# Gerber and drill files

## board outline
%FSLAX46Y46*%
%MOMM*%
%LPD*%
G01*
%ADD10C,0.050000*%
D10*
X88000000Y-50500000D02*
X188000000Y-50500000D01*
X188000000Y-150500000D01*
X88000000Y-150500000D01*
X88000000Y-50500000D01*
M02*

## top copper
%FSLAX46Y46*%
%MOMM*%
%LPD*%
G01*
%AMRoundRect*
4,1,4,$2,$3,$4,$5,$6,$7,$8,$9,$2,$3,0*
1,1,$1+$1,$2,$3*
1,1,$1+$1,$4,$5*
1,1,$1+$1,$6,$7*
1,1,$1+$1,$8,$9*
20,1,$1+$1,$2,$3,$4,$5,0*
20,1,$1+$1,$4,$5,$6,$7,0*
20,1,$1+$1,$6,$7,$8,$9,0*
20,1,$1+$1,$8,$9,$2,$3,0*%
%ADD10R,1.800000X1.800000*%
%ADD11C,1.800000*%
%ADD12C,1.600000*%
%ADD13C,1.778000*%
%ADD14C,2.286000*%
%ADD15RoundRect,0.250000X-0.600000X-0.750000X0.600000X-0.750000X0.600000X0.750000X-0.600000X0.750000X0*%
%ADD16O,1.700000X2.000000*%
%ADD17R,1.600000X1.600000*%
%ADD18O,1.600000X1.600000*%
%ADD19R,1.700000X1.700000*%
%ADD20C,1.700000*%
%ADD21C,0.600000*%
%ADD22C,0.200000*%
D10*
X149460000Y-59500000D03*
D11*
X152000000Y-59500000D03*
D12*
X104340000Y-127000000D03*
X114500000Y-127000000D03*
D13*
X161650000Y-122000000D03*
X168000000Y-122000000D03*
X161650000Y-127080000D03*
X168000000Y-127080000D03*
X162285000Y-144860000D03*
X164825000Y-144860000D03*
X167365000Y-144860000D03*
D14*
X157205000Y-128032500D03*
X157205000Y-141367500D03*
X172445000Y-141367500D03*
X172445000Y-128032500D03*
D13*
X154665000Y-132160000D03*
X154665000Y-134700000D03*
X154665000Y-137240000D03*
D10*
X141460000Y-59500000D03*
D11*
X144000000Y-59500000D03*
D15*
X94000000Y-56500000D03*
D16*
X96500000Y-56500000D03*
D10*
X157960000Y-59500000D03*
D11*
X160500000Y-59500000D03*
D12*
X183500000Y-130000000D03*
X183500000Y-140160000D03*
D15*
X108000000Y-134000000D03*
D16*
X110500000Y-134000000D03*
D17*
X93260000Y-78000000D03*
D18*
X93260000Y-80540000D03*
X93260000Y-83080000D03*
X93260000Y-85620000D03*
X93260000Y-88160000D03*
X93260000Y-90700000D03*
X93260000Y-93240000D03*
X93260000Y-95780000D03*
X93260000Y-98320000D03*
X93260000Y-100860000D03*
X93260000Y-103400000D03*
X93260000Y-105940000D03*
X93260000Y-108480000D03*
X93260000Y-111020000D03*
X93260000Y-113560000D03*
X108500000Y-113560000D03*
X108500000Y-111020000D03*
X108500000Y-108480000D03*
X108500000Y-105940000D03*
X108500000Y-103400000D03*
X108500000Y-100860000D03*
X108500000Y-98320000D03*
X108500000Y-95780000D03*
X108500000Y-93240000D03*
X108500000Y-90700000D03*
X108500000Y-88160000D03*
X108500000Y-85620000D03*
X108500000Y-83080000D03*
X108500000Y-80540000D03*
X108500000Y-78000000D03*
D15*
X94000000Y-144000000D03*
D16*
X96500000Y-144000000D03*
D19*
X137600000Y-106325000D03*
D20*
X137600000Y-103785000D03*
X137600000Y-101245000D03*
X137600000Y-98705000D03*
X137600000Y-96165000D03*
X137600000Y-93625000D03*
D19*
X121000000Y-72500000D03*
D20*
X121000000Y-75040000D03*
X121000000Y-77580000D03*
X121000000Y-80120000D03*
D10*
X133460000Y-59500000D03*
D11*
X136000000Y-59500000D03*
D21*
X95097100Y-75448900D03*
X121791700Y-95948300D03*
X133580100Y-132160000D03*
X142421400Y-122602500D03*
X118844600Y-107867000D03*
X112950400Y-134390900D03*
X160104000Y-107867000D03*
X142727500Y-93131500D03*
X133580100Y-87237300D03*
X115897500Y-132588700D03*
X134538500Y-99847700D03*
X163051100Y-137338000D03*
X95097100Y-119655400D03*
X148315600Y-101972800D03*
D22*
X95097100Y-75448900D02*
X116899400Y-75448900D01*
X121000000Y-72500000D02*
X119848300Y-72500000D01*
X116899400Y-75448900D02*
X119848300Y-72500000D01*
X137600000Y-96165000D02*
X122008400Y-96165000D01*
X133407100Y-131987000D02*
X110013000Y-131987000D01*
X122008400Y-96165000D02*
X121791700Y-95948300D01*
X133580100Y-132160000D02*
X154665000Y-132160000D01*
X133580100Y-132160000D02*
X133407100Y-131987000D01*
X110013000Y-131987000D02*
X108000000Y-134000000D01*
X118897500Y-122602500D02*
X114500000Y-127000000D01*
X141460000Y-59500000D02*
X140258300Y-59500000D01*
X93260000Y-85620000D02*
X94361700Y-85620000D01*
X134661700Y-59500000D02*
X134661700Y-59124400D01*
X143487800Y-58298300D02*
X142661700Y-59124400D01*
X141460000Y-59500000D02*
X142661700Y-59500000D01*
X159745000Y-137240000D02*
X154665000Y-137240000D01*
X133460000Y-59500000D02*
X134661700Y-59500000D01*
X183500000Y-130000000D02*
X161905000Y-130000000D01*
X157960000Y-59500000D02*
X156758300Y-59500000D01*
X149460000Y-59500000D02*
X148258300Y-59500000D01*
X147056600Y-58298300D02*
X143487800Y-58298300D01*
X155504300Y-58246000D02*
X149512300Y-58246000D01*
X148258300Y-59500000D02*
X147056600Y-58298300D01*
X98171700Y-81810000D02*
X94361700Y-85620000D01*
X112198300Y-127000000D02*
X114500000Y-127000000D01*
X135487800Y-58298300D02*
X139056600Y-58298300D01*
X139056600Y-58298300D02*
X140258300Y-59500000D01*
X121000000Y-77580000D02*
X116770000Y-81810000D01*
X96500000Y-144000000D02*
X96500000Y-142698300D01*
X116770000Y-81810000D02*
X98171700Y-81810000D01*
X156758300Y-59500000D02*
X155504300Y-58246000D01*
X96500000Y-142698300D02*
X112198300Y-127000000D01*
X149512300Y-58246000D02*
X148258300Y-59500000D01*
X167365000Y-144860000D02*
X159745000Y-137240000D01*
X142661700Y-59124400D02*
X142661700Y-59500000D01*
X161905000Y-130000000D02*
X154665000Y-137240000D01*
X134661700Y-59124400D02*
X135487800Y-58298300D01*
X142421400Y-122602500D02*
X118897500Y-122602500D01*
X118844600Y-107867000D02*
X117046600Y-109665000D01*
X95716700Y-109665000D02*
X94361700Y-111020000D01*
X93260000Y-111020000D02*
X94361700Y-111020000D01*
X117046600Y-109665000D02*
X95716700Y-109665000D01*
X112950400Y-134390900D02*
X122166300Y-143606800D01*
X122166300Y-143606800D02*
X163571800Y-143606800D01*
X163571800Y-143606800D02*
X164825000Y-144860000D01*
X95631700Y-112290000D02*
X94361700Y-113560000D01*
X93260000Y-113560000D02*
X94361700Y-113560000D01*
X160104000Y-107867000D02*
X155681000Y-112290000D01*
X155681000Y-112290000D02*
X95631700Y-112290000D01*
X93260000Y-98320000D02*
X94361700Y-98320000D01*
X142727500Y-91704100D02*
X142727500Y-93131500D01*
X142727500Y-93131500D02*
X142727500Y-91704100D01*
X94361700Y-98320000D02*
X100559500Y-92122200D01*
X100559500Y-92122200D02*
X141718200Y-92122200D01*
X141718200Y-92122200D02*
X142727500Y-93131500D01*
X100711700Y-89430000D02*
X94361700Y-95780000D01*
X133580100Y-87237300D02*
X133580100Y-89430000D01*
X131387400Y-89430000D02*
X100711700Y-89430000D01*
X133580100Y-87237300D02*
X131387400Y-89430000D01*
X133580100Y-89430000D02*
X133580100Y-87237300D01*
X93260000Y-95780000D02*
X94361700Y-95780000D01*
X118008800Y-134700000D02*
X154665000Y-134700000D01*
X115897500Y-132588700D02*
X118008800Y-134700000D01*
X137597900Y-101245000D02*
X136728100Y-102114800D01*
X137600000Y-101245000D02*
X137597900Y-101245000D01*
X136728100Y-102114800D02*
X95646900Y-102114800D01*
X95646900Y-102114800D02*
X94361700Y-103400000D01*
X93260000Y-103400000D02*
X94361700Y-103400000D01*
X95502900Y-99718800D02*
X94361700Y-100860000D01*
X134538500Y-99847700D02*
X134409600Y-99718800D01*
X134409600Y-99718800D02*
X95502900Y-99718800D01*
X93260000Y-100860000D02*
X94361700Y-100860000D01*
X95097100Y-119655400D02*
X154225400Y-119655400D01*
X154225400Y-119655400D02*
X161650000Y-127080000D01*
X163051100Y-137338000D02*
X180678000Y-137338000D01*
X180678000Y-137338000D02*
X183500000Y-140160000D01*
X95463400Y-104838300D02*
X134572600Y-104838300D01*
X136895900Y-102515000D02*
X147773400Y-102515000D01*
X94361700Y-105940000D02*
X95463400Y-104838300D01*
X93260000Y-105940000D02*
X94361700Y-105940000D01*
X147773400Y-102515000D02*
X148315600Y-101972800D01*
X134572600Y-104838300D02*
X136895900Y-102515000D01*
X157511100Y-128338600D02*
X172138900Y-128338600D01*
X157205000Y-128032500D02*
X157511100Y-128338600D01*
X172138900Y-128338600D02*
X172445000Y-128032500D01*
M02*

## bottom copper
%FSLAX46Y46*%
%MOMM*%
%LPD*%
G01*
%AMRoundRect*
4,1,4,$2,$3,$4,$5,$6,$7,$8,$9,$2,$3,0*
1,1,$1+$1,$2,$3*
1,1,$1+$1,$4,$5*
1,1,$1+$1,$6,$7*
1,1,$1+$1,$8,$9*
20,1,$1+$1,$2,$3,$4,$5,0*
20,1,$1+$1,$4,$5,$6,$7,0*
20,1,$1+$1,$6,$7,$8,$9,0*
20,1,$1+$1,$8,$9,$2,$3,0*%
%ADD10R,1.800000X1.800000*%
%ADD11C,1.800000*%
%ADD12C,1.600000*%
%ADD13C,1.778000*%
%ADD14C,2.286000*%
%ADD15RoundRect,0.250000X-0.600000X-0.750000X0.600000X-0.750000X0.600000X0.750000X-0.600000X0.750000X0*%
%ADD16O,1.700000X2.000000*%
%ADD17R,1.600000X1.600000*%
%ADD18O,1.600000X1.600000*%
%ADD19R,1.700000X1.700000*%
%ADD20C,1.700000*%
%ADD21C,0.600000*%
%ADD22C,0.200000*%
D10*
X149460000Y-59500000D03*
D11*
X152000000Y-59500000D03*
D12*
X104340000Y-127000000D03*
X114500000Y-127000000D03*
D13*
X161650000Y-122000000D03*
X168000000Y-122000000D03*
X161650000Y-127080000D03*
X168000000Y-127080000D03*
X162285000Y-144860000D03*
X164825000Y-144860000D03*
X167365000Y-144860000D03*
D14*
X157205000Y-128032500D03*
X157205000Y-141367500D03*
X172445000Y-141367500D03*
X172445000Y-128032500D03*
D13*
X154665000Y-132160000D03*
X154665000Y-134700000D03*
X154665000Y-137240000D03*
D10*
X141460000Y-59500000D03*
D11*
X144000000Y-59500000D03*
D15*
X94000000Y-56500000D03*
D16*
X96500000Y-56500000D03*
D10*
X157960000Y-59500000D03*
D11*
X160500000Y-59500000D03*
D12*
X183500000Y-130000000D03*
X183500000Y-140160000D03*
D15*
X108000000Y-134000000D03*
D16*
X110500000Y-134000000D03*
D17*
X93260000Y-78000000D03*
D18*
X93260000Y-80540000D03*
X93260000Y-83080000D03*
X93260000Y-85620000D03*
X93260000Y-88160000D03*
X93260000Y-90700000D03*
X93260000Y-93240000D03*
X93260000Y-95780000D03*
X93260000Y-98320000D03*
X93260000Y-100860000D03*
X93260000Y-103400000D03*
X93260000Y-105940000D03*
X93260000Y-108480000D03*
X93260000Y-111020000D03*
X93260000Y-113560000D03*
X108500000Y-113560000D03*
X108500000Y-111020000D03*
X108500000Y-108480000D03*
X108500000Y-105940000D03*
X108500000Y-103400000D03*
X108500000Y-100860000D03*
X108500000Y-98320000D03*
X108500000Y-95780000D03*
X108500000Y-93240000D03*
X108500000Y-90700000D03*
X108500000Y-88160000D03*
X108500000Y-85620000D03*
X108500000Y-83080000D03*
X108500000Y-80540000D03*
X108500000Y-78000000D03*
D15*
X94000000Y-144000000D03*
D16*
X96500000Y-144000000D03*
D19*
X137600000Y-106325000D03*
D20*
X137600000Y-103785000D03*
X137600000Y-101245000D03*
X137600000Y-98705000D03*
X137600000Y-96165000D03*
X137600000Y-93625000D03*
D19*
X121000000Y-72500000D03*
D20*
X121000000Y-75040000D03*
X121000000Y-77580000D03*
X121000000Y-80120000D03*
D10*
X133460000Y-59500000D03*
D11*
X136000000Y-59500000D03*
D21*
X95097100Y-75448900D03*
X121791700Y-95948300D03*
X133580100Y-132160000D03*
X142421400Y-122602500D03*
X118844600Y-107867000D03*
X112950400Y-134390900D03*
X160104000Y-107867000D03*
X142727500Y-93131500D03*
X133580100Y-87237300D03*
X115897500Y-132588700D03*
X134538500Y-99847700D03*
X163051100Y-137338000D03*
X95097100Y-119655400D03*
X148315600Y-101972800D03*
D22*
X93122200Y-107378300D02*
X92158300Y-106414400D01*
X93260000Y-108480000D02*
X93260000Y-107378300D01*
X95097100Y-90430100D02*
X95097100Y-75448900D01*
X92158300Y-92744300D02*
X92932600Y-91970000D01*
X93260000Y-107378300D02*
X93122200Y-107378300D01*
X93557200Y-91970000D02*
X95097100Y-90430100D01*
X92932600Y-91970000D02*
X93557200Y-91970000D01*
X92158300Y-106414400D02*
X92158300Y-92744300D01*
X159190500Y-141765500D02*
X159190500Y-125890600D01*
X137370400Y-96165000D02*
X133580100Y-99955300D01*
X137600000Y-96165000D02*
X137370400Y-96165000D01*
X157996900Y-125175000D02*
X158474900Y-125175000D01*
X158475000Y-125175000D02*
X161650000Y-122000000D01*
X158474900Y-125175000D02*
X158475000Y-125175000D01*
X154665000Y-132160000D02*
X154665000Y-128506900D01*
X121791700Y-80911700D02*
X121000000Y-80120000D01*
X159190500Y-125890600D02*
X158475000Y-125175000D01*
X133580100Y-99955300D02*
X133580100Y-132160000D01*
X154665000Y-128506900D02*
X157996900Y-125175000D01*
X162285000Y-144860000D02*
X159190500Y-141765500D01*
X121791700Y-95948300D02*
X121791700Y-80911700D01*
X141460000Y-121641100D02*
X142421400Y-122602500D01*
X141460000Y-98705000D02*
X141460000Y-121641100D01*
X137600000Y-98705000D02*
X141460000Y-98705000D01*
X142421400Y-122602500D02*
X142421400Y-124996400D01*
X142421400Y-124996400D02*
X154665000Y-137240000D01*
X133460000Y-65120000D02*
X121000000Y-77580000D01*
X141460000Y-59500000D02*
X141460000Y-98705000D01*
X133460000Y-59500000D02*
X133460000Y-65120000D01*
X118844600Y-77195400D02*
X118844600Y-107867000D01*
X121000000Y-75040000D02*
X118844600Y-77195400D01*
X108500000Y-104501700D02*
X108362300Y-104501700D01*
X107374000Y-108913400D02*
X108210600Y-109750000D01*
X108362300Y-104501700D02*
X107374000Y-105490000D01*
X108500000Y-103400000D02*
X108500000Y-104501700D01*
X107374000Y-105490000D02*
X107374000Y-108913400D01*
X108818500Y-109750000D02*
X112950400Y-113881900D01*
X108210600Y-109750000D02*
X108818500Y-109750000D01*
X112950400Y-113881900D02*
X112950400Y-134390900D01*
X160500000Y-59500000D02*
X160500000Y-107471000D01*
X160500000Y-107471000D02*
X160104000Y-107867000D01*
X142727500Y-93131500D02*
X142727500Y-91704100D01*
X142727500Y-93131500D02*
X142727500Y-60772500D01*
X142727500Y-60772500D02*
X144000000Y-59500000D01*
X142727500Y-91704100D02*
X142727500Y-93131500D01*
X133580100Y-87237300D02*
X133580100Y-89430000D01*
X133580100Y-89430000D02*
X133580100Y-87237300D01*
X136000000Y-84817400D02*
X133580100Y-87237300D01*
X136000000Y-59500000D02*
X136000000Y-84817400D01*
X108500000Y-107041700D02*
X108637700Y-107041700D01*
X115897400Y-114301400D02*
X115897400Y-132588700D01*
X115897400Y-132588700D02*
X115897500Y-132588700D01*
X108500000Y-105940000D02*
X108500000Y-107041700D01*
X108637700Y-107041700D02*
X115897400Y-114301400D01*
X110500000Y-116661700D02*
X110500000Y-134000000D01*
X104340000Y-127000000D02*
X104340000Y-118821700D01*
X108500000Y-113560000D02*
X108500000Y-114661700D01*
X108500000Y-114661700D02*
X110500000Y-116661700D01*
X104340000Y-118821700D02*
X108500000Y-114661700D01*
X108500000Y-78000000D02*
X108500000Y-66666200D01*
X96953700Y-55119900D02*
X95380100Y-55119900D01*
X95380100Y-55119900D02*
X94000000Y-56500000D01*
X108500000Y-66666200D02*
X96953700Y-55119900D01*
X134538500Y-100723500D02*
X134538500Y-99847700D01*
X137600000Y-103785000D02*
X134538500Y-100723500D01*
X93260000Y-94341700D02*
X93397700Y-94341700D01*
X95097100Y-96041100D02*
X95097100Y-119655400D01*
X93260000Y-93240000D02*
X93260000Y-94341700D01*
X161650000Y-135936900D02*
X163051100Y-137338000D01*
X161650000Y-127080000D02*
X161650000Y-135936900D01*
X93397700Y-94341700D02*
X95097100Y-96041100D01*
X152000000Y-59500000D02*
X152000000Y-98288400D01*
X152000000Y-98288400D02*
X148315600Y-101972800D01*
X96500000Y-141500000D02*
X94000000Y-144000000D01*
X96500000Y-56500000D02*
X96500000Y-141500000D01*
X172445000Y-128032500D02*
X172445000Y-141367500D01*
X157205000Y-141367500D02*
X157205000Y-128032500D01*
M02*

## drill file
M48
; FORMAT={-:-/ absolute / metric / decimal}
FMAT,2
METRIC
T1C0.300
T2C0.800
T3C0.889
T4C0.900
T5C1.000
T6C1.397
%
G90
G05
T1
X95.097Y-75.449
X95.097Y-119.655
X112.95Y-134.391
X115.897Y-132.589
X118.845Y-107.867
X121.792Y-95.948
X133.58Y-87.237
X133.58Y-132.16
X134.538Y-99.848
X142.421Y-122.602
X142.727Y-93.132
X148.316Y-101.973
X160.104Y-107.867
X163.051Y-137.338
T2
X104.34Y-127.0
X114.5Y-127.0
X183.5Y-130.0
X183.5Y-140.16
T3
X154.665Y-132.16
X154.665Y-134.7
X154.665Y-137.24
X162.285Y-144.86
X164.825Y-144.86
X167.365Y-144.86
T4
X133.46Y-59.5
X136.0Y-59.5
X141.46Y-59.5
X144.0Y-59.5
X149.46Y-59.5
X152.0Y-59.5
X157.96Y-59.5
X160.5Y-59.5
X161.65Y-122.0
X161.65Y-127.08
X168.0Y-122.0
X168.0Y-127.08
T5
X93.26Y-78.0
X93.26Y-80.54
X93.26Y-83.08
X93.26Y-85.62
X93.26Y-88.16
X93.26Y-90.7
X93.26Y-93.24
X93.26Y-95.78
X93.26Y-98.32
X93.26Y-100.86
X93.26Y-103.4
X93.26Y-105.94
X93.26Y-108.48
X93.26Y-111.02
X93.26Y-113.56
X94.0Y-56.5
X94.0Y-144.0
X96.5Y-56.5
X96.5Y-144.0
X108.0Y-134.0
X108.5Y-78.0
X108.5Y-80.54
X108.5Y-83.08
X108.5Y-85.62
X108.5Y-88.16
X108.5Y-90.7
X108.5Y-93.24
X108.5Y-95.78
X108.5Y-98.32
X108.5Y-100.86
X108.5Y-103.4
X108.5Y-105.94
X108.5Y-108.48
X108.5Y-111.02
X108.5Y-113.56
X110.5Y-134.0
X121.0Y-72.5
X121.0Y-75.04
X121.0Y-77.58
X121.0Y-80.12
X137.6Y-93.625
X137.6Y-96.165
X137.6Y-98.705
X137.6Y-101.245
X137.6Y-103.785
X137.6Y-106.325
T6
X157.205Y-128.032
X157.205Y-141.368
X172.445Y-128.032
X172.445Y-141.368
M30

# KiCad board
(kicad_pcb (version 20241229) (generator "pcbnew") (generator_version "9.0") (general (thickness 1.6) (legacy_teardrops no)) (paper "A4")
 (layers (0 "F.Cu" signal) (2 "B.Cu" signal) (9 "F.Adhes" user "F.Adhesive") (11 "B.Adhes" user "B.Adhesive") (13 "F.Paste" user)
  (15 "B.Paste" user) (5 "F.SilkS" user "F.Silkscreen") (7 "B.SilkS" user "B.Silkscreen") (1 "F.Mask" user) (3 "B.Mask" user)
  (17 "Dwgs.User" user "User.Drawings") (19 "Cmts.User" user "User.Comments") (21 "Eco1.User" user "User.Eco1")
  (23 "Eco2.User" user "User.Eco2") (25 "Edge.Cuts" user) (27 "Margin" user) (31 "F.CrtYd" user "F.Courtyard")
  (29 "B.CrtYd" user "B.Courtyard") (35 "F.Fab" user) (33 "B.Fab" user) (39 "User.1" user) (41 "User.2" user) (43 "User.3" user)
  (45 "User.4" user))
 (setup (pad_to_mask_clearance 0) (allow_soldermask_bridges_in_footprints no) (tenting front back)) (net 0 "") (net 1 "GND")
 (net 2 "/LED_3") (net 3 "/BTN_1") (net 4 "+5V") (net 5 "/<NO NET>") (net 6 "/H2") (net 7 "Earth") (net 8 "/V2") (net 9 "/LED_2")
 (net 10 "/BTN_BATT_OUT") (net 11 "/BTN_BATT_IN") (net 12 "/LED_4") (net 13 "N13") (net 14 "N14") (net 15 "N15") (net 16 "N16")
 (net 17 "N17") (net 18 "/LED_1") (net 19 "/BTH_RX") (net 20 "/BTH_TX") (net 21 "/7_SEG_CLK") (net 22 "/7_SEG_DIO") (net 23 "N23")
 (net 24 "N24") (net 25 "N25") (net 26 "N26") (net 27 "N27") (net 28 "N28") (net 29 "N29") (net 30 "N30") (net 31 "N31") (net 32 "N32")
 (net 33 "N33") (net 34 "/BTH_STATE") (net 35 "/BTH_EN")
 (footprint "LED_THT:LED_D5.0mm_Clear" (layer "F.Cu") (at 149.46 59.5)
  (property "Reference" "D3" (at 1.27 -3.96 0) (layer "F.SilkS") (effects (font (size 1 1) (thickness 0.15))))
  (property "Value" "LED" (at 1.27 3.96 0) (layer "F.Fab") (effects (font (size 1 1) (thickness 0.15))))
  (pad "1" thru_hole rect (at 0 0) (size 1.8 1.8) (drill 0.9) (layers "*.Cu" "*.Mask") (remove_unused_layers no) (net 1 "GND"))
  (pad "2" thru_hole circle (at 2.54 0) (size 1.8 1.8) (drill 0.9) (layers "*.Cu" "*.Mask") (remove_unused_layers no) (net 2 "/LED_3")))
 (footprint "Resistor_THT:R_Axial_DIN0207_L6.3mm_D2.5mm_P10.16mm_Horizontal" (layer "F.Cu") (at 104.34 127)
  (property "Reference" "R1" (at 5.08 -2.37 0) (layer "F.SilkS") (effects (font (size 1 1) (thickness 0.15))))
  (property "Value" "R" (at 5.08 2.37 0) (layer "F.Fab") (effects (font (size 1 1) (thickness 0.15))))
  (pad "1" thru_hole circle (at 0 0) (size 1.6 1.6) (drill 0.8) (layers "*.Cu" "*.Mask") (remove_unused_layers no) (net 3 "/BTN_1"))
  (pad "2" thru_hole circle (at 10.16 0) (size 1.6 1.6) (drill 0.8) (layers "*.Cu" "*.Mask") (remove_unused_layers no) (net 1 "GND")))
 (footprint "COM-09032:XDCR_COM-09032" (layer "F.Cu") (at 164.825 134.7)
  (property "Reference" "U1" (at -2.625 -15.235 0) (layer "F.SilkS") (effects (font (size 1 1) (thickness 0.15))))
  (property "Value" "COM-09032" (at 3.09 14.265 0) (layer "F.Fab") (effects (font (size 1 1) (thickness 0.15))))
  (pad "B1A" thru_hole circle (at -3.175 -12.7) (size 1.778 1.778) (drill 0.9) (layers "*.Cu" "*.Mask") (remove_unused_layers no)
   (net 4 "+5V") (solder_mask_margin 0.102))
  (pad "B1B" thru_hole circle (at 3.175 -12.7) (size 1.778 1.778) (drill 0.9) (layers "*.Cu" "*.Mask") (remove_unused_layers no)
   (solder_mask_margin 0.102))
  (pad "B2A" thru_hole circle (at -3.175 -7.62) (size 1.778 1.778) (drill 0.9) (layers "*.Cu" "*.Mask") (remove_unused_layers no)
   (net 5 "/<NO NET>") (solder_mask_margin 0.102))
  (pad "B2B" thru_hole circle (at 3.175 -7.62) (size 1.778 1.778) (drill 0.9) (layers "*.Cu" "*.Mask") (remove_unused_layers no)
   (solder_mask_margin 0.102))
  (pad "H1" thru_hole circle (at -2.54 10.16) (size 1.778 1.778) (drill 0.889) (layers "*.Cu" "*.Mask") (remove_unused_layers no)
   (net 4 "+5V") (solder_mask_margin 0.102))
  (pad "H2" thru_hole circle (at 0 10.16) (size 1.778 1.778) (drill 0.889) (layers "*.Cu" "*.Mask") (remove_unused_layers no) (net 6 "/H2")
   (solder_mask_margin 0.102))
  (pad "H3" thru_hole circle (at 2.54 10.16) (size 1.778 1.778) (drill 0.889) (layers "*.Cu" "*.Mask") (remove_unused_layers no)
   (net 1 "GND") (solder_mask_margin 0.102))
  (pad "S1" thru_hole circle (at -7.62 -6.6675) (size 2.286 2.286) (drill 1.397) (layers "*.Cu" "*.Mask") (remove_unused_layers no)
   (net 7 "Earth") (solder_mask_margin 0.102))
  (pad "S2" thru_hole circle (at -7.62 6.6675) (size 2.286 2.286) (drill 1.397) (layers "*.Cu" "*.Mask") (remove_unused_layers no)
   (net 7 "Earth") (solder_mask_margin 0.102))
  (pad "S3" thru_hole circle (at 7.62 6.6675) (size 2.286 2.286) (drill 1.397) (layers "*.Cu" "*.Mask") (remove_unused_layers no)
   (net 7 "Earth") (solder_mask_margin 0.102))
  (pad "S4" thru_hole circle (at 7.62 -6.6675) (size 2.286 2.286) (drill 1.397) (layers "*.Cu" "*.Mask") (remove_unused_layers no)
   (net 7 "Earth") (solder_mask_margin 0.102))
  (pad "V1" thru_hole circle (at -10.16 -2.54) (size 1.778 1.778) (drill 0.889) (layers "*.Cu" "*.Mask") (remove_unused_layers no)
   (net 4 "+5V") (solder_mask_margin 0.102))
  (pad "V2" thru_hole circle (at -10.16 0) (size 1.778 1.778) (drill 0.889) (layers "*.Cu" "*.Mask") (remove_unused_layers no) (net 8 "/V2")
   (solder_mask_margin 0.102))
  (pad "V3" thru_hole circle (at -10.16 2.54) (size 1.778 1.778) (drill 0.889) (layers "*.Cu" "*.Mask") (remove_unused_layers no)
   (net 1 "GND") (solder_mask_margin 0.102)))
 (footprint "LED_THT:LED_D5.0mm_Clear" (layer "F.Cu") (at 141.46 59.5)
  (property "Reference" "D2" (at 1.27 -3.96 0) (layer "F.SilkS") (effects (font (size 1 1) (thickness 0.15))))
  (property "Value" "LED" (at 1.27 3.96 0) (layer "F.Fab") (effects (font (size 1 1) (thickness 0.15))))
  (pad "1" thru_hole rect (at 0 0) (size 1.8 1.8) (drill 0.9) (layers "*.Cu" "*.Mask") (remove_unused_layers no) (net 1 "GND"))
  (pad "2" thru_hole circle (at 2.54 0) (size 1.8 1.8) (drill 0.9) (layers "*.Cu" "*.Mask") (remove_unused_layers no) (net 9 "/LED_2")))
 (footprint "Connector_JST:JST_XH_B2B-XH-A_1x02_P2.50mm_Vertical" (layer "F.Cu") (at 94 56.5)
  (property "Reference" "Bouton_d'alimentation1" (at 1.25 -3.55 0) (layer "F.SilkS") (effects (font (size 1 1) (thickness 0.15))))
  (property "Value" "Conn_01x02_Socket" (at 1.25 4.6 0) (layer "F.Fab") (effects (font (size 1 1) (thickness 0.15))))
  (pad "1" thru_hole roundrect (at 0 0) (size 1.7 2) (drill 1) (layers "*.Cu" "*.Mask") (remove_unused_layers no)
   (roundrect_rratio 0.147059) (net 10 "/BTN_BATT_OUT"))
  (pad "2" thru_hole oval (at 2.5 0) (size 1.7 2) (drill 1) (layers "*.Cu" "*.Mask") (remove_unused_layers no) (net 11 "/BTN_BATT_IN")))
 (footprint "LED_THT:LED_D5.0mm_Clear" (layer "F.Cu") (at 157.96 59.5)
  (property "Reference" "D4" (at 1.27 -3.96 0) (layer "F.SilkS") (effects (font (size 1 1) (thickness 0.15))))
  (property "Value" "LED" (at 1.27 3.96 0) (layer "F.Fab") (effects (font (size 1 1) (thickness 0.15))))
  (pad "1" thru_hole rect (at 0 0) (size 1.8 1.8) (drill 0.9) (layers "*.Cu" "*.Mask") (remove_unused_layers no) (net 1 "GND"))
  (pad "2" thru_hole circle (at 2.54 0) (size 1.8 1.8) (drill 0.9) (layers "*.Cu" "*.Mask") (remove_unused_layers no) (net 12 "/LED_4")))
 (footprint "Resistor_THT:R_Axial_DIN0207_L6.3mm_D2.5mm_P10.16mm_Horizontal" (layer "F.Cu") (at 183.5 130 -90)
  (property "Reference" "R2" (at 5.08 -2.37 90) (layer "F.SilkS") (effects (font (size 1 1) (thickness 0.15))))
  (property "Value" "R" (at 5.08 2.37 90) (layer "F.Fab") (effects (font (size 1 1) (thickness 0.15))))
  (pad "1" thru_hole circle (at 0 0 270) (size 1.6 1.6) (drill 0.8) (layers "*.Cu" "*.Mask") (remove_unused_layers no) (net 1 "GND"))
  (pad "2" thru_hole circle (at 10.16 0 270) (size 1.6 1.6) (drill 0.8) (layers "*.Cu" "*.Mask") (remove_unused_layers no)
   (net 5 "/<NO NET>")))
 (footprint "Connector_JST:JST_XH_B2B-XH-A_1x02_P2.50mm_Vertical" (layer "F.Cu") (at 108 134)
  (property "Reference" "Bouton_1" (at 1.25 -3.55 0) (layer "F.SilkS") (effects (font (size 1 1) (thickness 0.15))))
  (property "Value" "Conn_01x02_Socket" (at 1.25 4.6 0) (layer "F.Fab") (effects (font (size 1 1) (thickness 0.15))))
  (pad "1" thru_hole roundrect (at 0 0) (size 1.7 2) (drill 1) (layers "*.Cu" "*.Mask") (remove_unused_layers no)
   (roundrect_rratio 0.147059) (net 4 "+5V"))
  (pad "2" thru_hole oval (at 2.5 0) (size 1.7 2) (drill 1) (layers "*.Cu" "*.Mask") (remove_unused_layers no) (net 3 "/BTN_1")))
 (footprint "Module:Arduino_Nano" (layer "F.Cu") (at 93.26 78)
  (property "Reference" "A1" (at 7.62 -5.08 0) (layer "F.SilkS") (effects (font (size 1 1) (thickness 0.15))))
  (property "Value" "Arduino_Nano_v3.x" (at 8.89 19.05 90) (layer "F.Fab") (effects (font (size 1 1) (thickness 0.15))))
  (pad "1" thru_hole rect (at 0 0) (size 1.6 1.6) (drill 1) (layers "*.Cu" "*.Mask") (remove_unused_layers no) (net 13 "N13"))
  (pad "2" thru_hole oval (at 0 2.54) (size 1.6 1.6) (drill 1) (layers "*.Cu" "*.Mask") (remove_unused_layers no) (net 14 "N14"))
  (pad "3" thru_hole oval (at 0 5.08) (size 1.6 1.6) (drill 1) (layers "*.Cu" "*.Mask") (remove_unused_layers no) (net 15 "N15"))
  (pad "4" thru_hole oval (at 0 7.62) (size 1.6 1.6) (drill 1) (layers "*.Cu" "*.Mask") (remove_unused_layers no) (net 1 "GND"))
  (pad "5" thru_hole oval (at 0 10.16) (size 1.6 1.6) (drill 1) (layers "*.Cu" "*.Mask") (remove_unused_layers no) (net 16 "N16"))
  (pad "6" thru_hole oval (at 0 12.7) (size 1.6 1.6) (drill 1) (layers "*.Cu" "*.Mask") (remove_unused_layers no) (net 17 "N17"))
  (pad "7" thru_hole oval (at 0 15.24) (size 1.6 1.6) (drill 1) (layers "*.Cu" "*.Mask") (remove_unused_layers no) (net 5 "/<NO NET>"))
  (pad "8" thru_hole oval (at 0 17.78) (size 1.6 1.6) (drill 1) (layers "*.Cu" "*.Mask") (remove_unused_layers no) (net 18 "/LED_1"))
  (pad "9" thru_hole oval (at 0 20.32) (size 1.6 1.6) (drill 1) (layers "*.Cu" "*.Mask") (remove_unused_layers no) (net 9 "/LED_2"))
  (pad "10" thru_hole oval (at 0 22.86) (size 1.6 1.6) (drill 1) (layers "*.Cu" "*.Mask") (remove_unused_layers no) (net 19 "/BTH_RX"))
  (pad "11" thru_hole oval (at 0 25.4) (size 1.6 1.6) (drill 1) (layers "*.Cu" "*.Mask") (remove_unused_layers no) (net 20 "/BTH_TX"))
  (pad "12" thru_hole oval (at 0 27.94) (size 1.6 1.6) (drill 1) (layers "*.Cu" "*.Mask") (remove_unused_layers no) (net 2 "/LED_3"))
  (pad "13" thru_hole oval (at 0 30.48) (size 1.6 1.6) (drill 1) (layers "*.Cu" "*.Mask") (remove_unused_layers no) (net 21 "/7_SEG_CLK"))
  (pad "14" thru_hole oval (at 0 33.02) (size 1.6 1.6) (drill 1) (layers "*.Cu" "*.Mask") (remove_unused_layers no) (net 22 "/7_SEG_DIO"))
  (pad "15" thru_hole oval (at 0 35.56) (size 1.6 1.6) (drill 1) (layers "*.Cu" "*.Mask") (remove_unused_layers no) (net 12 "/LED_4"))
  (pad "16" thru_hole oval (at 15.24 35.56) (size 1.6 1.6) (drill 1) (layers "*.Cu" "*.Mask") (remove_unused_layers no) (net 3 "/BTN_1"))
  (pad "17" thru_hole oval (at 15.24 33.02) (size 1.6 1.6) (drill 1) (layers "*.Cu" "*.Mask") (remove_unused_layers no) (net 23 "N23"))
  (pad "18" thru_hole oval (at 15.24 30.48) (size 1.6 1.6) (drill 1) (layers "*.Cu" "*.Mask") (remove_unused_layers no) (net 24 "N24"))
  (pad "19" thru_hole oval (at 15.24 27.94) (size 1.6 1.6) (drill 1) (layers "*.Cu" "*.Mask") (remove_unused_layers no) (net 8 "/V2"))
  (pad "20" thru_hole oval (at 15.24 25.4) (size 1.6 1.6) (drill 1) (layers "*.Cu" "*.Mask") (remove_unused_layers no) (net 6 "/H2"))
  (pad "21" thru_hole oval (at 15.24 22.86) (size 1.6 1.6) (drill 1) (layers "*.Cu" "*.Mask") (remove_unused_layers no) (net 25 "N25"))
  (pad "22" thru_hole oval (at 15.24 20.32) (size 1.6 1.6) (drill 1) (layers "*.Cu" "*.Mask") (remove_unused_layers no) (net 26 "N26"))
  (pad "23" thru_hole oval (at 15.24 17.78) (size 1.6 1.6) (drill 1) (layers "*.Cu" "*.Mask") (remove_unused_layers no) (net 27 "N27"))
  (pad "24" thru_hole oval (at 15.24 15.24) (size 1.6 1.6) (drill 1) (layers "*.Cu" "*.Mask") (remove_unused_layers no) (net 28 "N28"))
  (pad "25" thru_hole oval (at 15.24 12.7) (size 1.6 1.6) (drill 1) (layers "*.Cu" "*.Mask") (remove_unused_layers no) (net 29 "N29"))
  (pad "26" thru_hole oval (at 15.24 10.16) (size 1.6 1.6) (drill 1) (layers "*.Cu" "*.Mask") (remove_unused_layers no) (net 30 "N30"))
  (pad "27" thru_hole oval (at 15.24 7.62) (size 1.6 1.6) (drill 1) (layers "*.Cu" "*.Mask") (remove_unused_layers no) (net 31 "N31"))
  (pad "28" thru_hole oval (at 15.24 5.08) (size 1.6 1.6) (drill 1) (layers "*.Cu" "*.Mask") (remove_unused_layers no) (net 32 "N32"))
  (pad "29" thru_hole oval (at 15.24 2.54) (size 1.6 1.6) (drill 1) (layers "*.Cu" "*.Mask") (remove_unused_layers no) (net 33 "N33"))
  (pad "30" thru_hole oval (at 15.24 0) (size 1.6 1.6) (drill 1) (layers "*.Cu" "*.Mask") (remove_unused_layers no) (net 10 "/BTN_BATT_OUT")))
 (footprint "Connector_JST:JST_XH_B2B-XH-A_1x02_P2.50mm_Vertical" (layer "F.Cu") (at 94 144)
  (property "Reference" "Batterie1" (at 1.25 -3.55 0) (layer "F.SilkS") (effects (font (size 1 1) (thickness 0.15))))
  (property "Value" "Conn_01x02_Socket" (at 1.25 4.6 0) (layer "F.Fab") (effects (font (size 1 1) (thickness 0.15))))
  (pad "1" thru_hole roundrect (at 0 0) (size 1.7 2) (drill 1) (layers "*.Cu" "*.Mask") (remove_unused_layers no)
   (roundrect_rratio 0.147059) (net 11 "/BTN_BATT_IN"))
  (pad "2" thru_hole oval (at 2.5 0) (size 1.7 2) (drill 1) (layers "*.Cu" "*.Mask") (remove_unused_layers no) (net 1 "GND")))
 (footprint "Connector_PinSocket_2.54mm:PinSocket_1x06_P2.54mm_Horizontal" (layer "F.Cu") (at 137.6 106.325 180)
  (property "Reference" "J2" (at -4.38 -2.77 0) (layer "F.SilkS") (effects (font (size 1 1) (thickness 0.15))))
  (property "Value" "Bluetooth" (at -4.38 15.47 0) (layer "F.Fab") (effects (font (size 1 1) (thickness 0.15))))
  (pad "1" thru_hole rect (at 0 0 180) (size 1.7 1.7) (drill 1) (layers "*.Cu" "*.Mask") (remove_unused_layers no) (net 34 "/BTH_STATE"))
  (pad "2" thru_hole circle (at 0 2.54 180) (size 1.7 1.7) (drill 1) (layers "*.Cu" "*.Mask") (remove_unused_layers no) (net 19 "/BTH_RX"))
  (pad "3" thru_hole circle (at 0 5.08 180) (size 1.7 1.7) (drill 1) (layers "*.Cu" "*.Mask") (remove_unused_layers no) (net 20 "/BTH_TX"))
  (pad "4" thru_hole circle (at 0 7.62 180) (size 1.7 1.7) (drill 1) (layers "*.Cu" "*.Mask") (remove_unused_layers no) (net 1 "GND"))
  (pad "5" thru_hole circle (at 0 10.16 180) (size 1.7 1.7) (drill 1) (layers "*.Cu" "*.Mask") (remove_unused_layers no) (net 4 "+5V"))
  (pad "6" thru_hole circle (at 0 12.7 180) (size 1.7 1.7) (drill 1) (layers "*.Cu" "*.Mask") (remove_unused_layers no) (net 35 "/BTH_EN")))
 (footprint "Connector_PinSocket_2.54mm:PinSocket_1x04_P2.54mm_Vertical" (layer "F.Cu") (at 121 72.5)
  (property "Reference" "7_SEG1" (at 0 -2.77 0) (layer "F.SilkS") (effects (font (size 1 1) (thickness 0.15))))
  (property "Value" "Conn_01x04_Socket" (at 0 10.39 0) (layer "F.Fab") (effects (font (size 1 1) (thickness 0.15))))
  (pad "1" thru_hole rect (at 0 0) (size 1.7 1.7) (drill 1) (layers "*.Cu" "*.Mask") (remove_unused_layers no) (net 21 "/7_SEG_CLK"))
  (pad "2" thru_hole circle (at 0 2.54) (size 1.7 1.7) (drill 1) (layers "*.Cu" "*.Mask") (remove_unused_layers no) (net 22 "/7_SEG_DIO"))
  (pad "3" thru_hole circle (at 0 5.08) (size 1.7 1.7) (drill 1) (layers "*.Cu" "*.Mask") (remove_unused_layers no) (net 1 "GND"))
  (pad "4" thru_hole circle (at 0 7.62) (size 1.7 1.7) (drill 1) (layers "*.Cu" "*.Mask") (remove_unused_layers no) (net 4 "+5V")))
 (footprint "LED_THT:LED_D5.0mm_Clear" (layer "F.Cu") (at 133.46 59.5)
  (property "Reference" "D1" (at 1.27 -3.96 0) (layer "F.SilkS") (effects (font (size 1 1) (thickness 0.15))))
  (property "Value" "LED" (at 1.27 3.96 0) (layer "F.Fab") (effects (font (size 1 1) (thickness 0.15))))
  (pad "1" thru_hole rect (at 0 0) (size 1.8 1.8) (drill 0.9) (layers "*.Cu" "*.Mask") (remove_unused_layers no) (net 1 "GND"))
  (pad "2" thru_hole circle (at 2.54 0) (size 1.8 1.8) (drill 0.9) (layers "*.Cu" "*.Mask") (remove_unused_layers no) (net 18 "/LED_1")))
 (gr_rect (start 88 50.5) (end 188 150.5) (stroke (width 0.05) (type solid)) (fill no) (layer "Edge.Cuts"))
 (segment (start 95.0971 75.4489) (end 116.8994 75.4489) (width 0.2) (layer "F.Cu") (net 21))
 (segment (start 121 72.5) (end 119.8483 72.5) (width 0.2) (layer "F.Cu") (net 21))
 (segment (start 116.8994 75.4489) (end 119.8483 72.5) (width 0.2) (layer "F.Cu") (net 21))
 (via (at 95.0971 75.4489) (size 0.6) (drill 0.3) (layers "F.Cu" "B.Cu") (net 21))
 (segment (start 93.1222 107.3783) (end 92.1583 106.4144) (width 0.2) (layer "B.Cu") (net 21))
 (segment (start 93.26 108.48) (end 93.26 107.3783) (width 0.2) (layer "B.Cu") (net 21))
 (segment (start 95.0971 90.4301) (end 95.0971 75.4489) (width 0.2) (layer "B.Cu") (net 21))
 (segment (start 92.1583 92.7443) (end 92.9326 91.97) (width 0.2) (layer "B.Cu") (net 21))
 (segment (start 93.26 107.3783) (end 93.1222 107.3783) (width 0.2) (layer "B.Cu") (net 21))
 (segment (start 93.5572 91.97) (end 95.0971 90.4301) (width 0.2) (layer "B.Cu") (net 21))
 (segment (start 92.9326 91.97) (end 93.5572 91.97) (width 0.2) (layer "B.Cu") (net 21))
 (segment (start 92.1583 106.4144) (end 92.1583 92.7443) (width 0.2) (layer "B.Cu") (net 21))
 (segment (start 137.6 96.165) (end 122.0084 96.165) (width 0.2) (layer "F.Cu") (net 4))
 (segment (start 133.4071 131.987) (end 110.013 131.987) (width 0.2) (layer "F.Cu") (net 4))
 (segment (start 122.0084 96.165) (end 121.7917 95.9483) (width 0.2) (layer "F.Cu") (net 4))
 (segment (start 133.5801 132.16) (end 154.665 132.16) (width 0.2) (layer "F.Cu") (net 4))
 (segment (start 133.5801 132.16) (end 133.4071 131.987) (width 0.2) (layer "F.Cu") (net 4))
 (segment (start 110.013 131.987) (end 108 134) (width 0.2) (layer "F.Cu") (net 4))
 (via (at 121.7917 95.9483) (size 0.6) (drill 0.3) (layers "F.Cu" "B.Cu") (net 4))
 (via (at 133.5801 132.16) (size 0.6) (drill 0.3) (layers "F.Cu" "B.Cu") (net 4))
 (segment (start 159.1905 141.7655) (end 159.1905 125.8906) (width 0.2) (layer "B.Cu") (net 4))
 (segment (start 137.3704 96.165) (end 133.5801 99.9553) (width 0.2) (layer "B.Cu") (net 4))
 (segment (start 137.6 96.165) (end 137.3704 96.165) (width 0.2) (layer "B.Cu") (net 4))
 (segment (start 157.9969 125.175) (end 158.4749 125.175) (width 0.2) (layer "B.Cu") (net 4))
 (segment (start 158.475 125.175) (end 161.65 122) (width 0.2) (layer "B.Cu") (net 4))
 (segment (start 158.4749 125.175) (end 158.475 125.175) (width 0.2) (layer "B.Cu") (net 4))
 (segment (start 154.665 132.16) (end 154.665 128.5069) (width 0.2) (layer "B.Cu") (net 4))
 (segment (start 121.7917 80.9117) (end 121 80.12) (width 0.2) (layer "B.Cu") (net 4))
 (segment (start 159.1905 125.8906) (end 158.475 125.175) (width 0.2) (layer "B.Cu") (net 4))
 (segment (start 133.5801 99.9553) (end 133.5801 132.16) (width 0.2) (layer "B.Cu") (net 4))
 (segment (start 154.665 128.5069) (end 157.9969 125.175) (width 0.2) (layer "B.Cu") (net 4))
 (segment (start 162.285 144.86) (end 159.1905 141.7655) (width 0.2) (layer "B.Cu") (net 4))
 (segment (start 121.7917 95.9483) (end 121.7917 80.9117) (width 0.2) (layer "B.Cu") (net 4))
 (segment (start 118.8975 122.6025) (end 114.5 127) (width 0.2) (layer "F.Cu") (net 1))
 (segment (start 141.46 59.5) (end 140.2583 59.5) (width 0.2) (layer "F.Cu") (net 1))
 (segment (start 93.26 85.62) (end 94.3617 85.62) (width 0.2) (layer "F.Cu") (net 1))
 (segment (start 134.6617 59.5) (end 134.6617 59.1244) (width 0.2) (layer "F.Cu") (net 1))
 (segment (start 143.4878 58.2983) (end 142.6617 59.1244) (width 0.2) (layer "F.Cu") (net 1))
 (segment (start 141.46 59.5) (end 142.6617 59.5) (width 0.2) (layer "F.Cu") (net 1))
 (segment (start 159.745 137.24) (end 154.665 137.24) (width 0.2) (layer "F.Cu") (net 1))
 (segment (start 133.46 59.5) (end 134.6617 59.5) (width 0.2) (layer "F.Cu") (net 1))
 (segment (start 183.5 130) (end 161.905 130) (width 0.2) (layer "F.Cu") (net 1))
 (segment (start 157.96 59.5) (end 156.7583 59.5) (width 0.2) (layer "F.Cu") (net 1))
 (segment (start 149.46 59.5) (end 148.2583 59.5) (width 0.2) (layer "F.Cu") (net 1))
 (segment (start 147.0566 58.2983) (end 143.4878 58.2983) (width 0.2) (layer "F.Cu") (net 1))
 (segment (start 155.5043 58.246) (end 149.5123 58.246) (width 0.2) (layer "F.Cu") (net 1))
 (segment (start 148.2583 59.5) (end 147.0566 58.2983) (width 0.2) (layer "F.Cu") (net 1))
 (segment (start 98.1717 81.81) (end 94.3617 85.62) (width 0.2) (layer "F.Cu") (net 1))
 (segment (start 112.1983 127) (end 114.5 127) (width 0.2) (layer "F.Cu") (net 1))
 (segment (start 135.4878 58.2983) (end 139.0566 58.2983) (width 0.2) (layer "F.Cu") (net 1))
 (segment (start 139.0566 58.2983) (end 140.2583 59.5) (width 0.2) (layer "F.Cu") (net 1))
 (segment (start 121 77.58) (end 116.77 81.81) (width 0.2) (layer "F.Cu") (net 1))
 (segment (start 96.5 144) (end 96.5 142.6983) (width 0.2) (layer "F.Cu") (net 1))
 (segment (start 116.77 81.81) (end 98.1717 81.81) (width 0.2) (layer "F.Cu") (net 1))
 (segment (start 156.7583 59.5) (end 155.5043 58.246) (width 0.2) (layer "F.Cu") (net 1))
 (segment (start 96.5 142.6983) (end 112.1983 127) (width 0.2) (layer "F.Cu") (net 1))
 (segment (start 149.5123 58.246) (end 148.2583 59.5) (width 0.2) (layer "F.Cu") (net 1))
 (segment (start 167.365 144.86) (end 159.745 137.24) (width 0.2) (layer "F.Cu") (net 1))
 (segment (start 142.6617 59.1244) (end 142.6617 59.5) (width 0.2) (layer "F.Cu") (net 1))
 (segment (start 161.905 130) (end 154.665 137.24) (width 0.2) (layer "F.Cu") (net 1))
 (segment (start 134.6617 59.1244) (end 135.4878 58.2983) (width 0.2) (layer "F.Cu") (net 1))
 (segment (start 142.4214 122.6025) (end 118.8975 122.6025) (width 0.2) (layer "F.Cu") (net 1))
 (via (at 142.4214 122.6025) (size 0.6) (drill 0.3) (layers "F.Cu" "B.Cu") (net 1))
 (segment (start 141.46 121.6411) (end 142.4214 122.6025) (width 0.2) (layer "B.Cu") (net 1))
 (segment (start 141.46 98.705) (end 141.46 121.6411) (width 0.2) (layer "B.Cu") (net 1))
 (segment (start 137.6 98.705) (end 141.46 98.705) (width 0.2) (layer "B.Cu") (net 1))
 (segment (start 142.4214 122.6025) (end 142.4214 124.9964) (width 0.2) (layer "B.Cu") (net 1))
 (segment (start 142.4214 124.9964) (end 154.665 137.24) (width 0.2) (layer "B.Cu") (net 1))
 (segment (start 133.46 65.12) (end 121 77.58) (width 0.2) (layer "B.Cu") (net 1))
 (segment (start 141.46 59.5) (end 141.46 98.705) (width 0.2) (layer "B.Cu") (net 1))
 (segment (start 133.46 59.5) (end 133.46 65.12) (width 0.2) (layer "B.Cu") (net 1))
 (segment (start 118.8446 107.867) (end 117.0466 109.665) (width 0.2) (layer "F.Cu") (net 22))
 (segment (start 95.7167 109.665) (end 94.3617 111.02) (width 0.2) (layer "F.Cu") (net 22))
 (segment (start 93.26 111.02) (end 94.3617 111.02) (width 0.2) (layer "F.Cu") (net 22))
 (segment (start 117.0466 109.665) (end 95.7167 109.665) (width 0.2) (layer "F.Cu") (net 22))
 (via (at 118.8446 107.867) (size 0.6) (drill 0.3) (layers "F.Cu" "B.Cu") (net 22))
 (segment (start 118.8446 77.1954) (end 118.8446 107.867) (width 0.2) (layer "B.Cu") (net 22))
 (segment (start 121 75.04) (end 118.8446 77.1954) (width 0.2) (layer "B.Cu") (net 22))
 (segment (start 112.9504 134.3909) (end 122.1663 143.6068) (width 0.2) (layer "F.Cu") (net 6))
 (segment (start 122.1663 143.6068) (end 163.5718 143.6068) (width 0.2) (layer "F.Cu") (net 6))
 (segment (start 163.5718 143.6068) (end 164.825 144.86) (width 0.2) (layer "F.Cu") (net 6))
 (via (at 112.9504 134.3909) (size 0.6) (drill 0.3) (layers "F.Cu" "B.Cu") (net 6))
 (segment (start 108.5 104.5017) (end 108.3623 104.5017) (width 0.2) (layer "B.Cu") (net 6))
 (segment (start 107.374 108.9134) (end 108.2106 109.75) (width 0.2) (layer "B.Cu") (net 6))
 (segment (start 108.3623 104.5017) (end 107.374 105.49) (width 0.2) (layer "B.Cu") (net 6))
 (segment (start 108.5 103.4) (end 108.5 104.5017) (width 0.2) (layer "B.Cu") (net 6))
 (segment (start 107.374 105.49) (end 107.374 108.9134) (width 0.2) (layer "B.Cu") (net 6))
 (segment (start 108.8185 109.75) (end 112.9504 113.8819) (width 0.2) (layer "B.Cu") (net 6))
 (segment (start 108.2106 109.75) (end 108.8185 109.75) (width 0.2) (layer "B.Cu") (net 6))
 (segment (start 112.9504 113.8819) (end 112.9504 134.3909) (width 0.2) (layer "B.Cu") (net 6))
 (segment (start 95.6317 112.29) (end 94.3617 113.56) (width 0.2) (layer "F.Cu") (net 12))
 (segment (start 93.26 113.56) (end 94.3617 113.56) (width 0.2) (layer "F.Cu") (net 12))
 (segment (start 160.104 107.867) (end 155.681 112.29) (width 0.2) (layer "F.Cu") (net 12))
 (segment (start 155.681 112.29) (end 95.6317 112.29) (width 0.2) (layer "F.Cu") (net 12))
 (via (at 160.104 107.867) (size 0.6) (drill 0.3) (layers "F.Cu" "B.Cu") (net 12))
 (segment (start 160.5 59.5) (end 160.5 107.471) (width 0.2) (layer "B.Cu") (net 12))
 (segment (start 160.5 107.471) (end 160.104 107.867) (width 0.2) (layer "B.Cu") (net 12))
 (segment (start 93.26 98.32) (end 94.3617 98.32) (width 0.2) (layer "F.Cu") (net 9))
 (segment (start 142.7275 91.7041) (end 142.7275 93.1315) (width 0.2) (layer "F.Cu") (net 9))
 (segment (start 142.7275 93.1315) (end 142.7275 91.7041) (width 0.2) (layer "F.Cu") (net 9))
 (segment (start 94.3617 98.32) (end 100.5595 92.1222) (width 0.2) (layer "F.Cu") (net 9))
 (segment (start 100.5595 92.1222) (end 141.7182 92.1222) (width 0.2) (layer "F.Cu") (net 9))
 (segment (start 141.7182 92.1222) (end 142.7275 93.1315) (width 0.2) (layer "F.Cu") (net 9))
 (via (at 142.7275 93.1315) (size 0.6) (drill 0.3) (layers "F.Cu" "B.Cu") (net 9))
 (segment (start 142.7275 93.1315) (end 142.7275 91.7041) (width 0.2) (layer "B.Cu") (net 9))
 (segment (start 142.7275 93.1315) (end 142.7275 60.7725) (width 0.2) (layer "B.Cu") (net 9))
 (segment (start 142.7275 60.7725) (end 144 59.5) (width 0.2) (layer "B.Cu") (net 9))
 (segment (start 142.7275 91.7041) (end 142.7275 93.1315) (width 0.2) (layer "B.Cu") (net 9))
 (segment (start 100.7117 89.43) (end 94.3617 95.78) (width 0.2) (layer "F.Cu") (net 18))
 (segment (start 133.5801 87.2373) (end 133.5801 89.43) (width 0.2) (layer "F.Cu") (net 18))
 (segment (start 131.3874 89.43) (end 100.7117 89.43) (width 0.2) (layer "F.Cu") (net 18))
 (segment (start 133.5801 87.2373) (end 131.3874 89.43) (width 0.2) (layer "F.Cu") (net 18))
 (segment (start 133.5801 89.43) (end 133.5801 87.2373) (width 0.2) (layer "F.Cu") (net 18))
 (segment (start 93.26 95.78) (end 94.3617 95.78) (width 0.2) (layer "F.Cu") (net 18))
 (via (at 133.5801 87.2373) (size 0.6) (drill 0.3) (layers "F.Cu" "B.Cu") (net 18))
 (segment (start 133.5801 87.2373) (end 133.5801 89.43) (width 0.2) (layer "B.Cu") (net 18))
 (segment (start 133.5801 89.43) (end 133.5801 87.2373) (width 0.2) (layer "B.Cu") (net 18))
 (segment (start 136 84.8174) (end 133.5801 87.2373) (width 0.2) (layer "B.Cu") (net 18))
 (segment (start 136 59.5) (end 136 84.8174) (width 0.2) (layer "B.Cu") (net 18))
 (segment (start 118.0088 134.7) (end 154.665 134.7) (width 0.2) (layer "F.Cu") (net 8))
 (segment (start 115.8975 132.5887) (end 118.0088 134.7) (width 0.2) (layer "F.Cu") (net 8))
 (via (at 115.8975 132.5887) (size 0.6) (drill 0.3) (layers "F.Cu" "B.Cu") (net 8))
 (segment (start 108.5 107.0417) (end 108.6377 107.0417) (width 0.2) (layer "B.Cu") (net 8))
 (segment (start 115.8974 114.3014) (end 115.8974 132.5887) (width 0.2) (layer "B.Cu") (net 8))
 (segment (start 115.8974 132.5887) (end 115.8975 132.5887) (width 0.2) (layer "B.Cu") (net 8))
 (segment (start 108.5 105.94) (end 108.5 107.0417) (width 0.2) (layer "B.Cu") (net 8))
 (segment (start 108.6377 107.0417) (end 115.8974 114.3014) (width 0.2) (layer "B.Cu") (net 8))
 (segment (start 137.5979 101.245) (end 136.7281 102.1148) (width 0.2) (layer "F.Cu") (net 20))
 (segment (start 137.6 101.245) (end 137.5979 101.245) (width 0.2) (layer "F.Cu") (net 20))
 (segment (start 136.7281 102.1148) (end 95.6469 102.1148) (width 0.2) (layer "F.Cu") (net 20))
 (segment (start 95.6469 102.1148) (end 94.3617 103.4) (width 0.2) (layer "F.Cu") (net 20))
 (segment (start 93.26 103.4) (end 94.3617 103.4) (width 0.2) (layer "F.Cu") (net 20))
 (segment (start 110.5 116.6617) (end 110.5 134) (width 0.2) (layer "B.Cu") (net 3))
 (segment (start 104.34 127) (end 104.34 118.8217) (width 0.2) (layer "B.Cu") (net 3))
 (segment (start 108.5 113.56) (end 108.5 114.6617) (width 0.2) (layer "B.Cu") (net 3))
 (segment (start 108.5 114.6617) (end 110.5 116.6617) (width 0.2) (layer "B.Cu") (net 3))
 (segment (start 104.34 118.8217) (end 108.5 114.6617) (width 0.2) (layer "B.Cu") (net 3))
 (segment (start 108.5 78) (end 108.5 66.6662) (width 0.2) (layer "B.Cu") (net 10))
 (segment (start 96.9537 55.1199) (end 95.3801 55.1199) (width 0.2) (layer "B.Cu") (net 10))
 (segment (start 95.3801 55.1199) (end 94 56.5) (width 0.2) (layer "B.Cu") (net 10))
 (segment (start 108.5 66.6662) (end 96.9537 55.1199) (width 0.2) (layer "B.Cu") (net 10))
 (segment (start 95.5029 99.7188) (end 94.3617 100.86) (width 0.2) (layer "F.Cu") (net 19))
 (segment (start 134.5385 99.8477) (end 134.4096 99.7188) (width 0.2) (layer "F.Cu") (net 19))
 (segment (start 134.4096 99.7188) (end 95.5029 99.7188) (width 0.2) (layer "F.Cu") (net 19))
 (segment (start 93.26 100.86) (end 94.3617 100.86) (width 0.2) (layer "F.Cu") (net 19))
 (via (at 134.5385 99.8477) (size 0.6) (drill 0.3) (layers "F.Cu" "B.Cu") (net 19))
 (segment (start 134.5385 100.7235) (end 134.5385 99.8477) (width 0.2) (layer "B.Cu") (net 19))
 (segment (start 137.6 103.785) (end 134.5385 100.7235) (width 0.2) (layer "B.Cu") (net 19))
 (segment (start 95.0971 119.6554) (end 154.2254 119.6554) (width 0.2) (layer "F.Cu") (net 5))
 (segment (start 154.2254 119.6554) (end 161.65 127.08) (width 0.2) (layer "F.Cu") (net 5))
 (segment (start 163.0511 137.338) (end 180.678 137.338) (width 0.2) (layer "F.Cu") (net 5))
 (segment (start 180.678 137.338) (end 183.5 140.16) (width 0.2) (layer "F.Cu") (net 5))
 (via (at 163.0511 137.338) (size 0.6) (drill 0.3) (layers "F.Cu" "B.Cu") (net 5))
 (via (at 95.0971 119.6554) (size 0.6) (drill 0.3) (layers "F.Cu" "B.Cu") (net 5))
 (segment (start 93.26 94.3417) (end 93.3977 94.3417) (width 0.2) (layer "B.Cu") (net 5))
 (segment (start 95.0971 96.0411) (end 95.0971 119.6554) (width 0.2) (layer "B.Cu") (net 5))
 (segment (start 93.26 93.24) (end 93.26 94.3417) (width 0.2) (layer "B.Cu") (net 5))
 (segment (start 161.65 135.9369) (end 163.0511 137.338) (width 0.2) (layer "B.Cu") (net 5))
 (segment (start 161.65 127.08) (end 161.65 135.9369) (width 0.2) (layer "B.Cu") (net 5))
 (segment (start 93.3977 94.3417) (end 95.0971 96.0411) (width 0.2) (layer "B.Cu") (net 5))
 (segment (start 95.4634 104.8383) (end 134.5726 104.8383) (width 0.2) (layer "F.Cu") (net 2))
 (segment (start 136.8959 102.515) (end 147.7734 102.515) (width 0.2) (layer "F.Cu") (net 2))
 (segment (start 94.3617 105.94) (end 95.4634 104.8383) (width 0.2) (layer "F.Cu") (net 2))
 (segment (start 93.26 105.94) (end 94.3617 105.94) (width 0.2) (layer "F.Cu") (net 2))
 (segment (start 147.7734 102.515) (end 148.3156 101.9728) (width 0.2) (layer "F.Cu") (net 2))
 (segment (start 134.5726 104.8383) (end 136.8959 102.515) (width 0.2) (layer "F.Cu") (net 2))
 (via (at 148.3156 101.9728) (size 0.6) (drill 0.3) (layers "F.Cu" "B.Cu") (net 2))
 (segment (start 152 59.5) (end 152 98.2884) (width 0.2) (layer "B.Cu") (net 2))
 (segment (start 152 98.2884) (end 148.3156 101.9728) (width 0.2) (layer "B.Cu") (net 2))
 (segment (start 96.5 141.5) (end 94 144) (width 0.2) (layer "B.Cu") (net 11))
 (segment (start 96.5 56.5) (end 96.5 141.5) (width 0.2) (layer "B.Cu") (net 11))
 (segment (start 157.5111 128.3386) (end 172.1389 128.3386) (width 0.2) (layer "F.Cu") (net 7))
 (segment (start 157.205 128.0325) (end 157.5111 128.3386) (width 0.2) (layer "F.Cu") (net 7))
 (segment (start 172.1389 128.3386) (end 172.445 128.0325) (width 0.2) (layer "F.Cu") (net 7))
 (segment (start 172.445 128.0325) (end 172.445 141.3675) (width 0.2) (layer "B.Cu") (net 7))
 (segment (start 157.205 141.3675) (end 157.205 128.0325) (width 0.2) (layer "B.Cu") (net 7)))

